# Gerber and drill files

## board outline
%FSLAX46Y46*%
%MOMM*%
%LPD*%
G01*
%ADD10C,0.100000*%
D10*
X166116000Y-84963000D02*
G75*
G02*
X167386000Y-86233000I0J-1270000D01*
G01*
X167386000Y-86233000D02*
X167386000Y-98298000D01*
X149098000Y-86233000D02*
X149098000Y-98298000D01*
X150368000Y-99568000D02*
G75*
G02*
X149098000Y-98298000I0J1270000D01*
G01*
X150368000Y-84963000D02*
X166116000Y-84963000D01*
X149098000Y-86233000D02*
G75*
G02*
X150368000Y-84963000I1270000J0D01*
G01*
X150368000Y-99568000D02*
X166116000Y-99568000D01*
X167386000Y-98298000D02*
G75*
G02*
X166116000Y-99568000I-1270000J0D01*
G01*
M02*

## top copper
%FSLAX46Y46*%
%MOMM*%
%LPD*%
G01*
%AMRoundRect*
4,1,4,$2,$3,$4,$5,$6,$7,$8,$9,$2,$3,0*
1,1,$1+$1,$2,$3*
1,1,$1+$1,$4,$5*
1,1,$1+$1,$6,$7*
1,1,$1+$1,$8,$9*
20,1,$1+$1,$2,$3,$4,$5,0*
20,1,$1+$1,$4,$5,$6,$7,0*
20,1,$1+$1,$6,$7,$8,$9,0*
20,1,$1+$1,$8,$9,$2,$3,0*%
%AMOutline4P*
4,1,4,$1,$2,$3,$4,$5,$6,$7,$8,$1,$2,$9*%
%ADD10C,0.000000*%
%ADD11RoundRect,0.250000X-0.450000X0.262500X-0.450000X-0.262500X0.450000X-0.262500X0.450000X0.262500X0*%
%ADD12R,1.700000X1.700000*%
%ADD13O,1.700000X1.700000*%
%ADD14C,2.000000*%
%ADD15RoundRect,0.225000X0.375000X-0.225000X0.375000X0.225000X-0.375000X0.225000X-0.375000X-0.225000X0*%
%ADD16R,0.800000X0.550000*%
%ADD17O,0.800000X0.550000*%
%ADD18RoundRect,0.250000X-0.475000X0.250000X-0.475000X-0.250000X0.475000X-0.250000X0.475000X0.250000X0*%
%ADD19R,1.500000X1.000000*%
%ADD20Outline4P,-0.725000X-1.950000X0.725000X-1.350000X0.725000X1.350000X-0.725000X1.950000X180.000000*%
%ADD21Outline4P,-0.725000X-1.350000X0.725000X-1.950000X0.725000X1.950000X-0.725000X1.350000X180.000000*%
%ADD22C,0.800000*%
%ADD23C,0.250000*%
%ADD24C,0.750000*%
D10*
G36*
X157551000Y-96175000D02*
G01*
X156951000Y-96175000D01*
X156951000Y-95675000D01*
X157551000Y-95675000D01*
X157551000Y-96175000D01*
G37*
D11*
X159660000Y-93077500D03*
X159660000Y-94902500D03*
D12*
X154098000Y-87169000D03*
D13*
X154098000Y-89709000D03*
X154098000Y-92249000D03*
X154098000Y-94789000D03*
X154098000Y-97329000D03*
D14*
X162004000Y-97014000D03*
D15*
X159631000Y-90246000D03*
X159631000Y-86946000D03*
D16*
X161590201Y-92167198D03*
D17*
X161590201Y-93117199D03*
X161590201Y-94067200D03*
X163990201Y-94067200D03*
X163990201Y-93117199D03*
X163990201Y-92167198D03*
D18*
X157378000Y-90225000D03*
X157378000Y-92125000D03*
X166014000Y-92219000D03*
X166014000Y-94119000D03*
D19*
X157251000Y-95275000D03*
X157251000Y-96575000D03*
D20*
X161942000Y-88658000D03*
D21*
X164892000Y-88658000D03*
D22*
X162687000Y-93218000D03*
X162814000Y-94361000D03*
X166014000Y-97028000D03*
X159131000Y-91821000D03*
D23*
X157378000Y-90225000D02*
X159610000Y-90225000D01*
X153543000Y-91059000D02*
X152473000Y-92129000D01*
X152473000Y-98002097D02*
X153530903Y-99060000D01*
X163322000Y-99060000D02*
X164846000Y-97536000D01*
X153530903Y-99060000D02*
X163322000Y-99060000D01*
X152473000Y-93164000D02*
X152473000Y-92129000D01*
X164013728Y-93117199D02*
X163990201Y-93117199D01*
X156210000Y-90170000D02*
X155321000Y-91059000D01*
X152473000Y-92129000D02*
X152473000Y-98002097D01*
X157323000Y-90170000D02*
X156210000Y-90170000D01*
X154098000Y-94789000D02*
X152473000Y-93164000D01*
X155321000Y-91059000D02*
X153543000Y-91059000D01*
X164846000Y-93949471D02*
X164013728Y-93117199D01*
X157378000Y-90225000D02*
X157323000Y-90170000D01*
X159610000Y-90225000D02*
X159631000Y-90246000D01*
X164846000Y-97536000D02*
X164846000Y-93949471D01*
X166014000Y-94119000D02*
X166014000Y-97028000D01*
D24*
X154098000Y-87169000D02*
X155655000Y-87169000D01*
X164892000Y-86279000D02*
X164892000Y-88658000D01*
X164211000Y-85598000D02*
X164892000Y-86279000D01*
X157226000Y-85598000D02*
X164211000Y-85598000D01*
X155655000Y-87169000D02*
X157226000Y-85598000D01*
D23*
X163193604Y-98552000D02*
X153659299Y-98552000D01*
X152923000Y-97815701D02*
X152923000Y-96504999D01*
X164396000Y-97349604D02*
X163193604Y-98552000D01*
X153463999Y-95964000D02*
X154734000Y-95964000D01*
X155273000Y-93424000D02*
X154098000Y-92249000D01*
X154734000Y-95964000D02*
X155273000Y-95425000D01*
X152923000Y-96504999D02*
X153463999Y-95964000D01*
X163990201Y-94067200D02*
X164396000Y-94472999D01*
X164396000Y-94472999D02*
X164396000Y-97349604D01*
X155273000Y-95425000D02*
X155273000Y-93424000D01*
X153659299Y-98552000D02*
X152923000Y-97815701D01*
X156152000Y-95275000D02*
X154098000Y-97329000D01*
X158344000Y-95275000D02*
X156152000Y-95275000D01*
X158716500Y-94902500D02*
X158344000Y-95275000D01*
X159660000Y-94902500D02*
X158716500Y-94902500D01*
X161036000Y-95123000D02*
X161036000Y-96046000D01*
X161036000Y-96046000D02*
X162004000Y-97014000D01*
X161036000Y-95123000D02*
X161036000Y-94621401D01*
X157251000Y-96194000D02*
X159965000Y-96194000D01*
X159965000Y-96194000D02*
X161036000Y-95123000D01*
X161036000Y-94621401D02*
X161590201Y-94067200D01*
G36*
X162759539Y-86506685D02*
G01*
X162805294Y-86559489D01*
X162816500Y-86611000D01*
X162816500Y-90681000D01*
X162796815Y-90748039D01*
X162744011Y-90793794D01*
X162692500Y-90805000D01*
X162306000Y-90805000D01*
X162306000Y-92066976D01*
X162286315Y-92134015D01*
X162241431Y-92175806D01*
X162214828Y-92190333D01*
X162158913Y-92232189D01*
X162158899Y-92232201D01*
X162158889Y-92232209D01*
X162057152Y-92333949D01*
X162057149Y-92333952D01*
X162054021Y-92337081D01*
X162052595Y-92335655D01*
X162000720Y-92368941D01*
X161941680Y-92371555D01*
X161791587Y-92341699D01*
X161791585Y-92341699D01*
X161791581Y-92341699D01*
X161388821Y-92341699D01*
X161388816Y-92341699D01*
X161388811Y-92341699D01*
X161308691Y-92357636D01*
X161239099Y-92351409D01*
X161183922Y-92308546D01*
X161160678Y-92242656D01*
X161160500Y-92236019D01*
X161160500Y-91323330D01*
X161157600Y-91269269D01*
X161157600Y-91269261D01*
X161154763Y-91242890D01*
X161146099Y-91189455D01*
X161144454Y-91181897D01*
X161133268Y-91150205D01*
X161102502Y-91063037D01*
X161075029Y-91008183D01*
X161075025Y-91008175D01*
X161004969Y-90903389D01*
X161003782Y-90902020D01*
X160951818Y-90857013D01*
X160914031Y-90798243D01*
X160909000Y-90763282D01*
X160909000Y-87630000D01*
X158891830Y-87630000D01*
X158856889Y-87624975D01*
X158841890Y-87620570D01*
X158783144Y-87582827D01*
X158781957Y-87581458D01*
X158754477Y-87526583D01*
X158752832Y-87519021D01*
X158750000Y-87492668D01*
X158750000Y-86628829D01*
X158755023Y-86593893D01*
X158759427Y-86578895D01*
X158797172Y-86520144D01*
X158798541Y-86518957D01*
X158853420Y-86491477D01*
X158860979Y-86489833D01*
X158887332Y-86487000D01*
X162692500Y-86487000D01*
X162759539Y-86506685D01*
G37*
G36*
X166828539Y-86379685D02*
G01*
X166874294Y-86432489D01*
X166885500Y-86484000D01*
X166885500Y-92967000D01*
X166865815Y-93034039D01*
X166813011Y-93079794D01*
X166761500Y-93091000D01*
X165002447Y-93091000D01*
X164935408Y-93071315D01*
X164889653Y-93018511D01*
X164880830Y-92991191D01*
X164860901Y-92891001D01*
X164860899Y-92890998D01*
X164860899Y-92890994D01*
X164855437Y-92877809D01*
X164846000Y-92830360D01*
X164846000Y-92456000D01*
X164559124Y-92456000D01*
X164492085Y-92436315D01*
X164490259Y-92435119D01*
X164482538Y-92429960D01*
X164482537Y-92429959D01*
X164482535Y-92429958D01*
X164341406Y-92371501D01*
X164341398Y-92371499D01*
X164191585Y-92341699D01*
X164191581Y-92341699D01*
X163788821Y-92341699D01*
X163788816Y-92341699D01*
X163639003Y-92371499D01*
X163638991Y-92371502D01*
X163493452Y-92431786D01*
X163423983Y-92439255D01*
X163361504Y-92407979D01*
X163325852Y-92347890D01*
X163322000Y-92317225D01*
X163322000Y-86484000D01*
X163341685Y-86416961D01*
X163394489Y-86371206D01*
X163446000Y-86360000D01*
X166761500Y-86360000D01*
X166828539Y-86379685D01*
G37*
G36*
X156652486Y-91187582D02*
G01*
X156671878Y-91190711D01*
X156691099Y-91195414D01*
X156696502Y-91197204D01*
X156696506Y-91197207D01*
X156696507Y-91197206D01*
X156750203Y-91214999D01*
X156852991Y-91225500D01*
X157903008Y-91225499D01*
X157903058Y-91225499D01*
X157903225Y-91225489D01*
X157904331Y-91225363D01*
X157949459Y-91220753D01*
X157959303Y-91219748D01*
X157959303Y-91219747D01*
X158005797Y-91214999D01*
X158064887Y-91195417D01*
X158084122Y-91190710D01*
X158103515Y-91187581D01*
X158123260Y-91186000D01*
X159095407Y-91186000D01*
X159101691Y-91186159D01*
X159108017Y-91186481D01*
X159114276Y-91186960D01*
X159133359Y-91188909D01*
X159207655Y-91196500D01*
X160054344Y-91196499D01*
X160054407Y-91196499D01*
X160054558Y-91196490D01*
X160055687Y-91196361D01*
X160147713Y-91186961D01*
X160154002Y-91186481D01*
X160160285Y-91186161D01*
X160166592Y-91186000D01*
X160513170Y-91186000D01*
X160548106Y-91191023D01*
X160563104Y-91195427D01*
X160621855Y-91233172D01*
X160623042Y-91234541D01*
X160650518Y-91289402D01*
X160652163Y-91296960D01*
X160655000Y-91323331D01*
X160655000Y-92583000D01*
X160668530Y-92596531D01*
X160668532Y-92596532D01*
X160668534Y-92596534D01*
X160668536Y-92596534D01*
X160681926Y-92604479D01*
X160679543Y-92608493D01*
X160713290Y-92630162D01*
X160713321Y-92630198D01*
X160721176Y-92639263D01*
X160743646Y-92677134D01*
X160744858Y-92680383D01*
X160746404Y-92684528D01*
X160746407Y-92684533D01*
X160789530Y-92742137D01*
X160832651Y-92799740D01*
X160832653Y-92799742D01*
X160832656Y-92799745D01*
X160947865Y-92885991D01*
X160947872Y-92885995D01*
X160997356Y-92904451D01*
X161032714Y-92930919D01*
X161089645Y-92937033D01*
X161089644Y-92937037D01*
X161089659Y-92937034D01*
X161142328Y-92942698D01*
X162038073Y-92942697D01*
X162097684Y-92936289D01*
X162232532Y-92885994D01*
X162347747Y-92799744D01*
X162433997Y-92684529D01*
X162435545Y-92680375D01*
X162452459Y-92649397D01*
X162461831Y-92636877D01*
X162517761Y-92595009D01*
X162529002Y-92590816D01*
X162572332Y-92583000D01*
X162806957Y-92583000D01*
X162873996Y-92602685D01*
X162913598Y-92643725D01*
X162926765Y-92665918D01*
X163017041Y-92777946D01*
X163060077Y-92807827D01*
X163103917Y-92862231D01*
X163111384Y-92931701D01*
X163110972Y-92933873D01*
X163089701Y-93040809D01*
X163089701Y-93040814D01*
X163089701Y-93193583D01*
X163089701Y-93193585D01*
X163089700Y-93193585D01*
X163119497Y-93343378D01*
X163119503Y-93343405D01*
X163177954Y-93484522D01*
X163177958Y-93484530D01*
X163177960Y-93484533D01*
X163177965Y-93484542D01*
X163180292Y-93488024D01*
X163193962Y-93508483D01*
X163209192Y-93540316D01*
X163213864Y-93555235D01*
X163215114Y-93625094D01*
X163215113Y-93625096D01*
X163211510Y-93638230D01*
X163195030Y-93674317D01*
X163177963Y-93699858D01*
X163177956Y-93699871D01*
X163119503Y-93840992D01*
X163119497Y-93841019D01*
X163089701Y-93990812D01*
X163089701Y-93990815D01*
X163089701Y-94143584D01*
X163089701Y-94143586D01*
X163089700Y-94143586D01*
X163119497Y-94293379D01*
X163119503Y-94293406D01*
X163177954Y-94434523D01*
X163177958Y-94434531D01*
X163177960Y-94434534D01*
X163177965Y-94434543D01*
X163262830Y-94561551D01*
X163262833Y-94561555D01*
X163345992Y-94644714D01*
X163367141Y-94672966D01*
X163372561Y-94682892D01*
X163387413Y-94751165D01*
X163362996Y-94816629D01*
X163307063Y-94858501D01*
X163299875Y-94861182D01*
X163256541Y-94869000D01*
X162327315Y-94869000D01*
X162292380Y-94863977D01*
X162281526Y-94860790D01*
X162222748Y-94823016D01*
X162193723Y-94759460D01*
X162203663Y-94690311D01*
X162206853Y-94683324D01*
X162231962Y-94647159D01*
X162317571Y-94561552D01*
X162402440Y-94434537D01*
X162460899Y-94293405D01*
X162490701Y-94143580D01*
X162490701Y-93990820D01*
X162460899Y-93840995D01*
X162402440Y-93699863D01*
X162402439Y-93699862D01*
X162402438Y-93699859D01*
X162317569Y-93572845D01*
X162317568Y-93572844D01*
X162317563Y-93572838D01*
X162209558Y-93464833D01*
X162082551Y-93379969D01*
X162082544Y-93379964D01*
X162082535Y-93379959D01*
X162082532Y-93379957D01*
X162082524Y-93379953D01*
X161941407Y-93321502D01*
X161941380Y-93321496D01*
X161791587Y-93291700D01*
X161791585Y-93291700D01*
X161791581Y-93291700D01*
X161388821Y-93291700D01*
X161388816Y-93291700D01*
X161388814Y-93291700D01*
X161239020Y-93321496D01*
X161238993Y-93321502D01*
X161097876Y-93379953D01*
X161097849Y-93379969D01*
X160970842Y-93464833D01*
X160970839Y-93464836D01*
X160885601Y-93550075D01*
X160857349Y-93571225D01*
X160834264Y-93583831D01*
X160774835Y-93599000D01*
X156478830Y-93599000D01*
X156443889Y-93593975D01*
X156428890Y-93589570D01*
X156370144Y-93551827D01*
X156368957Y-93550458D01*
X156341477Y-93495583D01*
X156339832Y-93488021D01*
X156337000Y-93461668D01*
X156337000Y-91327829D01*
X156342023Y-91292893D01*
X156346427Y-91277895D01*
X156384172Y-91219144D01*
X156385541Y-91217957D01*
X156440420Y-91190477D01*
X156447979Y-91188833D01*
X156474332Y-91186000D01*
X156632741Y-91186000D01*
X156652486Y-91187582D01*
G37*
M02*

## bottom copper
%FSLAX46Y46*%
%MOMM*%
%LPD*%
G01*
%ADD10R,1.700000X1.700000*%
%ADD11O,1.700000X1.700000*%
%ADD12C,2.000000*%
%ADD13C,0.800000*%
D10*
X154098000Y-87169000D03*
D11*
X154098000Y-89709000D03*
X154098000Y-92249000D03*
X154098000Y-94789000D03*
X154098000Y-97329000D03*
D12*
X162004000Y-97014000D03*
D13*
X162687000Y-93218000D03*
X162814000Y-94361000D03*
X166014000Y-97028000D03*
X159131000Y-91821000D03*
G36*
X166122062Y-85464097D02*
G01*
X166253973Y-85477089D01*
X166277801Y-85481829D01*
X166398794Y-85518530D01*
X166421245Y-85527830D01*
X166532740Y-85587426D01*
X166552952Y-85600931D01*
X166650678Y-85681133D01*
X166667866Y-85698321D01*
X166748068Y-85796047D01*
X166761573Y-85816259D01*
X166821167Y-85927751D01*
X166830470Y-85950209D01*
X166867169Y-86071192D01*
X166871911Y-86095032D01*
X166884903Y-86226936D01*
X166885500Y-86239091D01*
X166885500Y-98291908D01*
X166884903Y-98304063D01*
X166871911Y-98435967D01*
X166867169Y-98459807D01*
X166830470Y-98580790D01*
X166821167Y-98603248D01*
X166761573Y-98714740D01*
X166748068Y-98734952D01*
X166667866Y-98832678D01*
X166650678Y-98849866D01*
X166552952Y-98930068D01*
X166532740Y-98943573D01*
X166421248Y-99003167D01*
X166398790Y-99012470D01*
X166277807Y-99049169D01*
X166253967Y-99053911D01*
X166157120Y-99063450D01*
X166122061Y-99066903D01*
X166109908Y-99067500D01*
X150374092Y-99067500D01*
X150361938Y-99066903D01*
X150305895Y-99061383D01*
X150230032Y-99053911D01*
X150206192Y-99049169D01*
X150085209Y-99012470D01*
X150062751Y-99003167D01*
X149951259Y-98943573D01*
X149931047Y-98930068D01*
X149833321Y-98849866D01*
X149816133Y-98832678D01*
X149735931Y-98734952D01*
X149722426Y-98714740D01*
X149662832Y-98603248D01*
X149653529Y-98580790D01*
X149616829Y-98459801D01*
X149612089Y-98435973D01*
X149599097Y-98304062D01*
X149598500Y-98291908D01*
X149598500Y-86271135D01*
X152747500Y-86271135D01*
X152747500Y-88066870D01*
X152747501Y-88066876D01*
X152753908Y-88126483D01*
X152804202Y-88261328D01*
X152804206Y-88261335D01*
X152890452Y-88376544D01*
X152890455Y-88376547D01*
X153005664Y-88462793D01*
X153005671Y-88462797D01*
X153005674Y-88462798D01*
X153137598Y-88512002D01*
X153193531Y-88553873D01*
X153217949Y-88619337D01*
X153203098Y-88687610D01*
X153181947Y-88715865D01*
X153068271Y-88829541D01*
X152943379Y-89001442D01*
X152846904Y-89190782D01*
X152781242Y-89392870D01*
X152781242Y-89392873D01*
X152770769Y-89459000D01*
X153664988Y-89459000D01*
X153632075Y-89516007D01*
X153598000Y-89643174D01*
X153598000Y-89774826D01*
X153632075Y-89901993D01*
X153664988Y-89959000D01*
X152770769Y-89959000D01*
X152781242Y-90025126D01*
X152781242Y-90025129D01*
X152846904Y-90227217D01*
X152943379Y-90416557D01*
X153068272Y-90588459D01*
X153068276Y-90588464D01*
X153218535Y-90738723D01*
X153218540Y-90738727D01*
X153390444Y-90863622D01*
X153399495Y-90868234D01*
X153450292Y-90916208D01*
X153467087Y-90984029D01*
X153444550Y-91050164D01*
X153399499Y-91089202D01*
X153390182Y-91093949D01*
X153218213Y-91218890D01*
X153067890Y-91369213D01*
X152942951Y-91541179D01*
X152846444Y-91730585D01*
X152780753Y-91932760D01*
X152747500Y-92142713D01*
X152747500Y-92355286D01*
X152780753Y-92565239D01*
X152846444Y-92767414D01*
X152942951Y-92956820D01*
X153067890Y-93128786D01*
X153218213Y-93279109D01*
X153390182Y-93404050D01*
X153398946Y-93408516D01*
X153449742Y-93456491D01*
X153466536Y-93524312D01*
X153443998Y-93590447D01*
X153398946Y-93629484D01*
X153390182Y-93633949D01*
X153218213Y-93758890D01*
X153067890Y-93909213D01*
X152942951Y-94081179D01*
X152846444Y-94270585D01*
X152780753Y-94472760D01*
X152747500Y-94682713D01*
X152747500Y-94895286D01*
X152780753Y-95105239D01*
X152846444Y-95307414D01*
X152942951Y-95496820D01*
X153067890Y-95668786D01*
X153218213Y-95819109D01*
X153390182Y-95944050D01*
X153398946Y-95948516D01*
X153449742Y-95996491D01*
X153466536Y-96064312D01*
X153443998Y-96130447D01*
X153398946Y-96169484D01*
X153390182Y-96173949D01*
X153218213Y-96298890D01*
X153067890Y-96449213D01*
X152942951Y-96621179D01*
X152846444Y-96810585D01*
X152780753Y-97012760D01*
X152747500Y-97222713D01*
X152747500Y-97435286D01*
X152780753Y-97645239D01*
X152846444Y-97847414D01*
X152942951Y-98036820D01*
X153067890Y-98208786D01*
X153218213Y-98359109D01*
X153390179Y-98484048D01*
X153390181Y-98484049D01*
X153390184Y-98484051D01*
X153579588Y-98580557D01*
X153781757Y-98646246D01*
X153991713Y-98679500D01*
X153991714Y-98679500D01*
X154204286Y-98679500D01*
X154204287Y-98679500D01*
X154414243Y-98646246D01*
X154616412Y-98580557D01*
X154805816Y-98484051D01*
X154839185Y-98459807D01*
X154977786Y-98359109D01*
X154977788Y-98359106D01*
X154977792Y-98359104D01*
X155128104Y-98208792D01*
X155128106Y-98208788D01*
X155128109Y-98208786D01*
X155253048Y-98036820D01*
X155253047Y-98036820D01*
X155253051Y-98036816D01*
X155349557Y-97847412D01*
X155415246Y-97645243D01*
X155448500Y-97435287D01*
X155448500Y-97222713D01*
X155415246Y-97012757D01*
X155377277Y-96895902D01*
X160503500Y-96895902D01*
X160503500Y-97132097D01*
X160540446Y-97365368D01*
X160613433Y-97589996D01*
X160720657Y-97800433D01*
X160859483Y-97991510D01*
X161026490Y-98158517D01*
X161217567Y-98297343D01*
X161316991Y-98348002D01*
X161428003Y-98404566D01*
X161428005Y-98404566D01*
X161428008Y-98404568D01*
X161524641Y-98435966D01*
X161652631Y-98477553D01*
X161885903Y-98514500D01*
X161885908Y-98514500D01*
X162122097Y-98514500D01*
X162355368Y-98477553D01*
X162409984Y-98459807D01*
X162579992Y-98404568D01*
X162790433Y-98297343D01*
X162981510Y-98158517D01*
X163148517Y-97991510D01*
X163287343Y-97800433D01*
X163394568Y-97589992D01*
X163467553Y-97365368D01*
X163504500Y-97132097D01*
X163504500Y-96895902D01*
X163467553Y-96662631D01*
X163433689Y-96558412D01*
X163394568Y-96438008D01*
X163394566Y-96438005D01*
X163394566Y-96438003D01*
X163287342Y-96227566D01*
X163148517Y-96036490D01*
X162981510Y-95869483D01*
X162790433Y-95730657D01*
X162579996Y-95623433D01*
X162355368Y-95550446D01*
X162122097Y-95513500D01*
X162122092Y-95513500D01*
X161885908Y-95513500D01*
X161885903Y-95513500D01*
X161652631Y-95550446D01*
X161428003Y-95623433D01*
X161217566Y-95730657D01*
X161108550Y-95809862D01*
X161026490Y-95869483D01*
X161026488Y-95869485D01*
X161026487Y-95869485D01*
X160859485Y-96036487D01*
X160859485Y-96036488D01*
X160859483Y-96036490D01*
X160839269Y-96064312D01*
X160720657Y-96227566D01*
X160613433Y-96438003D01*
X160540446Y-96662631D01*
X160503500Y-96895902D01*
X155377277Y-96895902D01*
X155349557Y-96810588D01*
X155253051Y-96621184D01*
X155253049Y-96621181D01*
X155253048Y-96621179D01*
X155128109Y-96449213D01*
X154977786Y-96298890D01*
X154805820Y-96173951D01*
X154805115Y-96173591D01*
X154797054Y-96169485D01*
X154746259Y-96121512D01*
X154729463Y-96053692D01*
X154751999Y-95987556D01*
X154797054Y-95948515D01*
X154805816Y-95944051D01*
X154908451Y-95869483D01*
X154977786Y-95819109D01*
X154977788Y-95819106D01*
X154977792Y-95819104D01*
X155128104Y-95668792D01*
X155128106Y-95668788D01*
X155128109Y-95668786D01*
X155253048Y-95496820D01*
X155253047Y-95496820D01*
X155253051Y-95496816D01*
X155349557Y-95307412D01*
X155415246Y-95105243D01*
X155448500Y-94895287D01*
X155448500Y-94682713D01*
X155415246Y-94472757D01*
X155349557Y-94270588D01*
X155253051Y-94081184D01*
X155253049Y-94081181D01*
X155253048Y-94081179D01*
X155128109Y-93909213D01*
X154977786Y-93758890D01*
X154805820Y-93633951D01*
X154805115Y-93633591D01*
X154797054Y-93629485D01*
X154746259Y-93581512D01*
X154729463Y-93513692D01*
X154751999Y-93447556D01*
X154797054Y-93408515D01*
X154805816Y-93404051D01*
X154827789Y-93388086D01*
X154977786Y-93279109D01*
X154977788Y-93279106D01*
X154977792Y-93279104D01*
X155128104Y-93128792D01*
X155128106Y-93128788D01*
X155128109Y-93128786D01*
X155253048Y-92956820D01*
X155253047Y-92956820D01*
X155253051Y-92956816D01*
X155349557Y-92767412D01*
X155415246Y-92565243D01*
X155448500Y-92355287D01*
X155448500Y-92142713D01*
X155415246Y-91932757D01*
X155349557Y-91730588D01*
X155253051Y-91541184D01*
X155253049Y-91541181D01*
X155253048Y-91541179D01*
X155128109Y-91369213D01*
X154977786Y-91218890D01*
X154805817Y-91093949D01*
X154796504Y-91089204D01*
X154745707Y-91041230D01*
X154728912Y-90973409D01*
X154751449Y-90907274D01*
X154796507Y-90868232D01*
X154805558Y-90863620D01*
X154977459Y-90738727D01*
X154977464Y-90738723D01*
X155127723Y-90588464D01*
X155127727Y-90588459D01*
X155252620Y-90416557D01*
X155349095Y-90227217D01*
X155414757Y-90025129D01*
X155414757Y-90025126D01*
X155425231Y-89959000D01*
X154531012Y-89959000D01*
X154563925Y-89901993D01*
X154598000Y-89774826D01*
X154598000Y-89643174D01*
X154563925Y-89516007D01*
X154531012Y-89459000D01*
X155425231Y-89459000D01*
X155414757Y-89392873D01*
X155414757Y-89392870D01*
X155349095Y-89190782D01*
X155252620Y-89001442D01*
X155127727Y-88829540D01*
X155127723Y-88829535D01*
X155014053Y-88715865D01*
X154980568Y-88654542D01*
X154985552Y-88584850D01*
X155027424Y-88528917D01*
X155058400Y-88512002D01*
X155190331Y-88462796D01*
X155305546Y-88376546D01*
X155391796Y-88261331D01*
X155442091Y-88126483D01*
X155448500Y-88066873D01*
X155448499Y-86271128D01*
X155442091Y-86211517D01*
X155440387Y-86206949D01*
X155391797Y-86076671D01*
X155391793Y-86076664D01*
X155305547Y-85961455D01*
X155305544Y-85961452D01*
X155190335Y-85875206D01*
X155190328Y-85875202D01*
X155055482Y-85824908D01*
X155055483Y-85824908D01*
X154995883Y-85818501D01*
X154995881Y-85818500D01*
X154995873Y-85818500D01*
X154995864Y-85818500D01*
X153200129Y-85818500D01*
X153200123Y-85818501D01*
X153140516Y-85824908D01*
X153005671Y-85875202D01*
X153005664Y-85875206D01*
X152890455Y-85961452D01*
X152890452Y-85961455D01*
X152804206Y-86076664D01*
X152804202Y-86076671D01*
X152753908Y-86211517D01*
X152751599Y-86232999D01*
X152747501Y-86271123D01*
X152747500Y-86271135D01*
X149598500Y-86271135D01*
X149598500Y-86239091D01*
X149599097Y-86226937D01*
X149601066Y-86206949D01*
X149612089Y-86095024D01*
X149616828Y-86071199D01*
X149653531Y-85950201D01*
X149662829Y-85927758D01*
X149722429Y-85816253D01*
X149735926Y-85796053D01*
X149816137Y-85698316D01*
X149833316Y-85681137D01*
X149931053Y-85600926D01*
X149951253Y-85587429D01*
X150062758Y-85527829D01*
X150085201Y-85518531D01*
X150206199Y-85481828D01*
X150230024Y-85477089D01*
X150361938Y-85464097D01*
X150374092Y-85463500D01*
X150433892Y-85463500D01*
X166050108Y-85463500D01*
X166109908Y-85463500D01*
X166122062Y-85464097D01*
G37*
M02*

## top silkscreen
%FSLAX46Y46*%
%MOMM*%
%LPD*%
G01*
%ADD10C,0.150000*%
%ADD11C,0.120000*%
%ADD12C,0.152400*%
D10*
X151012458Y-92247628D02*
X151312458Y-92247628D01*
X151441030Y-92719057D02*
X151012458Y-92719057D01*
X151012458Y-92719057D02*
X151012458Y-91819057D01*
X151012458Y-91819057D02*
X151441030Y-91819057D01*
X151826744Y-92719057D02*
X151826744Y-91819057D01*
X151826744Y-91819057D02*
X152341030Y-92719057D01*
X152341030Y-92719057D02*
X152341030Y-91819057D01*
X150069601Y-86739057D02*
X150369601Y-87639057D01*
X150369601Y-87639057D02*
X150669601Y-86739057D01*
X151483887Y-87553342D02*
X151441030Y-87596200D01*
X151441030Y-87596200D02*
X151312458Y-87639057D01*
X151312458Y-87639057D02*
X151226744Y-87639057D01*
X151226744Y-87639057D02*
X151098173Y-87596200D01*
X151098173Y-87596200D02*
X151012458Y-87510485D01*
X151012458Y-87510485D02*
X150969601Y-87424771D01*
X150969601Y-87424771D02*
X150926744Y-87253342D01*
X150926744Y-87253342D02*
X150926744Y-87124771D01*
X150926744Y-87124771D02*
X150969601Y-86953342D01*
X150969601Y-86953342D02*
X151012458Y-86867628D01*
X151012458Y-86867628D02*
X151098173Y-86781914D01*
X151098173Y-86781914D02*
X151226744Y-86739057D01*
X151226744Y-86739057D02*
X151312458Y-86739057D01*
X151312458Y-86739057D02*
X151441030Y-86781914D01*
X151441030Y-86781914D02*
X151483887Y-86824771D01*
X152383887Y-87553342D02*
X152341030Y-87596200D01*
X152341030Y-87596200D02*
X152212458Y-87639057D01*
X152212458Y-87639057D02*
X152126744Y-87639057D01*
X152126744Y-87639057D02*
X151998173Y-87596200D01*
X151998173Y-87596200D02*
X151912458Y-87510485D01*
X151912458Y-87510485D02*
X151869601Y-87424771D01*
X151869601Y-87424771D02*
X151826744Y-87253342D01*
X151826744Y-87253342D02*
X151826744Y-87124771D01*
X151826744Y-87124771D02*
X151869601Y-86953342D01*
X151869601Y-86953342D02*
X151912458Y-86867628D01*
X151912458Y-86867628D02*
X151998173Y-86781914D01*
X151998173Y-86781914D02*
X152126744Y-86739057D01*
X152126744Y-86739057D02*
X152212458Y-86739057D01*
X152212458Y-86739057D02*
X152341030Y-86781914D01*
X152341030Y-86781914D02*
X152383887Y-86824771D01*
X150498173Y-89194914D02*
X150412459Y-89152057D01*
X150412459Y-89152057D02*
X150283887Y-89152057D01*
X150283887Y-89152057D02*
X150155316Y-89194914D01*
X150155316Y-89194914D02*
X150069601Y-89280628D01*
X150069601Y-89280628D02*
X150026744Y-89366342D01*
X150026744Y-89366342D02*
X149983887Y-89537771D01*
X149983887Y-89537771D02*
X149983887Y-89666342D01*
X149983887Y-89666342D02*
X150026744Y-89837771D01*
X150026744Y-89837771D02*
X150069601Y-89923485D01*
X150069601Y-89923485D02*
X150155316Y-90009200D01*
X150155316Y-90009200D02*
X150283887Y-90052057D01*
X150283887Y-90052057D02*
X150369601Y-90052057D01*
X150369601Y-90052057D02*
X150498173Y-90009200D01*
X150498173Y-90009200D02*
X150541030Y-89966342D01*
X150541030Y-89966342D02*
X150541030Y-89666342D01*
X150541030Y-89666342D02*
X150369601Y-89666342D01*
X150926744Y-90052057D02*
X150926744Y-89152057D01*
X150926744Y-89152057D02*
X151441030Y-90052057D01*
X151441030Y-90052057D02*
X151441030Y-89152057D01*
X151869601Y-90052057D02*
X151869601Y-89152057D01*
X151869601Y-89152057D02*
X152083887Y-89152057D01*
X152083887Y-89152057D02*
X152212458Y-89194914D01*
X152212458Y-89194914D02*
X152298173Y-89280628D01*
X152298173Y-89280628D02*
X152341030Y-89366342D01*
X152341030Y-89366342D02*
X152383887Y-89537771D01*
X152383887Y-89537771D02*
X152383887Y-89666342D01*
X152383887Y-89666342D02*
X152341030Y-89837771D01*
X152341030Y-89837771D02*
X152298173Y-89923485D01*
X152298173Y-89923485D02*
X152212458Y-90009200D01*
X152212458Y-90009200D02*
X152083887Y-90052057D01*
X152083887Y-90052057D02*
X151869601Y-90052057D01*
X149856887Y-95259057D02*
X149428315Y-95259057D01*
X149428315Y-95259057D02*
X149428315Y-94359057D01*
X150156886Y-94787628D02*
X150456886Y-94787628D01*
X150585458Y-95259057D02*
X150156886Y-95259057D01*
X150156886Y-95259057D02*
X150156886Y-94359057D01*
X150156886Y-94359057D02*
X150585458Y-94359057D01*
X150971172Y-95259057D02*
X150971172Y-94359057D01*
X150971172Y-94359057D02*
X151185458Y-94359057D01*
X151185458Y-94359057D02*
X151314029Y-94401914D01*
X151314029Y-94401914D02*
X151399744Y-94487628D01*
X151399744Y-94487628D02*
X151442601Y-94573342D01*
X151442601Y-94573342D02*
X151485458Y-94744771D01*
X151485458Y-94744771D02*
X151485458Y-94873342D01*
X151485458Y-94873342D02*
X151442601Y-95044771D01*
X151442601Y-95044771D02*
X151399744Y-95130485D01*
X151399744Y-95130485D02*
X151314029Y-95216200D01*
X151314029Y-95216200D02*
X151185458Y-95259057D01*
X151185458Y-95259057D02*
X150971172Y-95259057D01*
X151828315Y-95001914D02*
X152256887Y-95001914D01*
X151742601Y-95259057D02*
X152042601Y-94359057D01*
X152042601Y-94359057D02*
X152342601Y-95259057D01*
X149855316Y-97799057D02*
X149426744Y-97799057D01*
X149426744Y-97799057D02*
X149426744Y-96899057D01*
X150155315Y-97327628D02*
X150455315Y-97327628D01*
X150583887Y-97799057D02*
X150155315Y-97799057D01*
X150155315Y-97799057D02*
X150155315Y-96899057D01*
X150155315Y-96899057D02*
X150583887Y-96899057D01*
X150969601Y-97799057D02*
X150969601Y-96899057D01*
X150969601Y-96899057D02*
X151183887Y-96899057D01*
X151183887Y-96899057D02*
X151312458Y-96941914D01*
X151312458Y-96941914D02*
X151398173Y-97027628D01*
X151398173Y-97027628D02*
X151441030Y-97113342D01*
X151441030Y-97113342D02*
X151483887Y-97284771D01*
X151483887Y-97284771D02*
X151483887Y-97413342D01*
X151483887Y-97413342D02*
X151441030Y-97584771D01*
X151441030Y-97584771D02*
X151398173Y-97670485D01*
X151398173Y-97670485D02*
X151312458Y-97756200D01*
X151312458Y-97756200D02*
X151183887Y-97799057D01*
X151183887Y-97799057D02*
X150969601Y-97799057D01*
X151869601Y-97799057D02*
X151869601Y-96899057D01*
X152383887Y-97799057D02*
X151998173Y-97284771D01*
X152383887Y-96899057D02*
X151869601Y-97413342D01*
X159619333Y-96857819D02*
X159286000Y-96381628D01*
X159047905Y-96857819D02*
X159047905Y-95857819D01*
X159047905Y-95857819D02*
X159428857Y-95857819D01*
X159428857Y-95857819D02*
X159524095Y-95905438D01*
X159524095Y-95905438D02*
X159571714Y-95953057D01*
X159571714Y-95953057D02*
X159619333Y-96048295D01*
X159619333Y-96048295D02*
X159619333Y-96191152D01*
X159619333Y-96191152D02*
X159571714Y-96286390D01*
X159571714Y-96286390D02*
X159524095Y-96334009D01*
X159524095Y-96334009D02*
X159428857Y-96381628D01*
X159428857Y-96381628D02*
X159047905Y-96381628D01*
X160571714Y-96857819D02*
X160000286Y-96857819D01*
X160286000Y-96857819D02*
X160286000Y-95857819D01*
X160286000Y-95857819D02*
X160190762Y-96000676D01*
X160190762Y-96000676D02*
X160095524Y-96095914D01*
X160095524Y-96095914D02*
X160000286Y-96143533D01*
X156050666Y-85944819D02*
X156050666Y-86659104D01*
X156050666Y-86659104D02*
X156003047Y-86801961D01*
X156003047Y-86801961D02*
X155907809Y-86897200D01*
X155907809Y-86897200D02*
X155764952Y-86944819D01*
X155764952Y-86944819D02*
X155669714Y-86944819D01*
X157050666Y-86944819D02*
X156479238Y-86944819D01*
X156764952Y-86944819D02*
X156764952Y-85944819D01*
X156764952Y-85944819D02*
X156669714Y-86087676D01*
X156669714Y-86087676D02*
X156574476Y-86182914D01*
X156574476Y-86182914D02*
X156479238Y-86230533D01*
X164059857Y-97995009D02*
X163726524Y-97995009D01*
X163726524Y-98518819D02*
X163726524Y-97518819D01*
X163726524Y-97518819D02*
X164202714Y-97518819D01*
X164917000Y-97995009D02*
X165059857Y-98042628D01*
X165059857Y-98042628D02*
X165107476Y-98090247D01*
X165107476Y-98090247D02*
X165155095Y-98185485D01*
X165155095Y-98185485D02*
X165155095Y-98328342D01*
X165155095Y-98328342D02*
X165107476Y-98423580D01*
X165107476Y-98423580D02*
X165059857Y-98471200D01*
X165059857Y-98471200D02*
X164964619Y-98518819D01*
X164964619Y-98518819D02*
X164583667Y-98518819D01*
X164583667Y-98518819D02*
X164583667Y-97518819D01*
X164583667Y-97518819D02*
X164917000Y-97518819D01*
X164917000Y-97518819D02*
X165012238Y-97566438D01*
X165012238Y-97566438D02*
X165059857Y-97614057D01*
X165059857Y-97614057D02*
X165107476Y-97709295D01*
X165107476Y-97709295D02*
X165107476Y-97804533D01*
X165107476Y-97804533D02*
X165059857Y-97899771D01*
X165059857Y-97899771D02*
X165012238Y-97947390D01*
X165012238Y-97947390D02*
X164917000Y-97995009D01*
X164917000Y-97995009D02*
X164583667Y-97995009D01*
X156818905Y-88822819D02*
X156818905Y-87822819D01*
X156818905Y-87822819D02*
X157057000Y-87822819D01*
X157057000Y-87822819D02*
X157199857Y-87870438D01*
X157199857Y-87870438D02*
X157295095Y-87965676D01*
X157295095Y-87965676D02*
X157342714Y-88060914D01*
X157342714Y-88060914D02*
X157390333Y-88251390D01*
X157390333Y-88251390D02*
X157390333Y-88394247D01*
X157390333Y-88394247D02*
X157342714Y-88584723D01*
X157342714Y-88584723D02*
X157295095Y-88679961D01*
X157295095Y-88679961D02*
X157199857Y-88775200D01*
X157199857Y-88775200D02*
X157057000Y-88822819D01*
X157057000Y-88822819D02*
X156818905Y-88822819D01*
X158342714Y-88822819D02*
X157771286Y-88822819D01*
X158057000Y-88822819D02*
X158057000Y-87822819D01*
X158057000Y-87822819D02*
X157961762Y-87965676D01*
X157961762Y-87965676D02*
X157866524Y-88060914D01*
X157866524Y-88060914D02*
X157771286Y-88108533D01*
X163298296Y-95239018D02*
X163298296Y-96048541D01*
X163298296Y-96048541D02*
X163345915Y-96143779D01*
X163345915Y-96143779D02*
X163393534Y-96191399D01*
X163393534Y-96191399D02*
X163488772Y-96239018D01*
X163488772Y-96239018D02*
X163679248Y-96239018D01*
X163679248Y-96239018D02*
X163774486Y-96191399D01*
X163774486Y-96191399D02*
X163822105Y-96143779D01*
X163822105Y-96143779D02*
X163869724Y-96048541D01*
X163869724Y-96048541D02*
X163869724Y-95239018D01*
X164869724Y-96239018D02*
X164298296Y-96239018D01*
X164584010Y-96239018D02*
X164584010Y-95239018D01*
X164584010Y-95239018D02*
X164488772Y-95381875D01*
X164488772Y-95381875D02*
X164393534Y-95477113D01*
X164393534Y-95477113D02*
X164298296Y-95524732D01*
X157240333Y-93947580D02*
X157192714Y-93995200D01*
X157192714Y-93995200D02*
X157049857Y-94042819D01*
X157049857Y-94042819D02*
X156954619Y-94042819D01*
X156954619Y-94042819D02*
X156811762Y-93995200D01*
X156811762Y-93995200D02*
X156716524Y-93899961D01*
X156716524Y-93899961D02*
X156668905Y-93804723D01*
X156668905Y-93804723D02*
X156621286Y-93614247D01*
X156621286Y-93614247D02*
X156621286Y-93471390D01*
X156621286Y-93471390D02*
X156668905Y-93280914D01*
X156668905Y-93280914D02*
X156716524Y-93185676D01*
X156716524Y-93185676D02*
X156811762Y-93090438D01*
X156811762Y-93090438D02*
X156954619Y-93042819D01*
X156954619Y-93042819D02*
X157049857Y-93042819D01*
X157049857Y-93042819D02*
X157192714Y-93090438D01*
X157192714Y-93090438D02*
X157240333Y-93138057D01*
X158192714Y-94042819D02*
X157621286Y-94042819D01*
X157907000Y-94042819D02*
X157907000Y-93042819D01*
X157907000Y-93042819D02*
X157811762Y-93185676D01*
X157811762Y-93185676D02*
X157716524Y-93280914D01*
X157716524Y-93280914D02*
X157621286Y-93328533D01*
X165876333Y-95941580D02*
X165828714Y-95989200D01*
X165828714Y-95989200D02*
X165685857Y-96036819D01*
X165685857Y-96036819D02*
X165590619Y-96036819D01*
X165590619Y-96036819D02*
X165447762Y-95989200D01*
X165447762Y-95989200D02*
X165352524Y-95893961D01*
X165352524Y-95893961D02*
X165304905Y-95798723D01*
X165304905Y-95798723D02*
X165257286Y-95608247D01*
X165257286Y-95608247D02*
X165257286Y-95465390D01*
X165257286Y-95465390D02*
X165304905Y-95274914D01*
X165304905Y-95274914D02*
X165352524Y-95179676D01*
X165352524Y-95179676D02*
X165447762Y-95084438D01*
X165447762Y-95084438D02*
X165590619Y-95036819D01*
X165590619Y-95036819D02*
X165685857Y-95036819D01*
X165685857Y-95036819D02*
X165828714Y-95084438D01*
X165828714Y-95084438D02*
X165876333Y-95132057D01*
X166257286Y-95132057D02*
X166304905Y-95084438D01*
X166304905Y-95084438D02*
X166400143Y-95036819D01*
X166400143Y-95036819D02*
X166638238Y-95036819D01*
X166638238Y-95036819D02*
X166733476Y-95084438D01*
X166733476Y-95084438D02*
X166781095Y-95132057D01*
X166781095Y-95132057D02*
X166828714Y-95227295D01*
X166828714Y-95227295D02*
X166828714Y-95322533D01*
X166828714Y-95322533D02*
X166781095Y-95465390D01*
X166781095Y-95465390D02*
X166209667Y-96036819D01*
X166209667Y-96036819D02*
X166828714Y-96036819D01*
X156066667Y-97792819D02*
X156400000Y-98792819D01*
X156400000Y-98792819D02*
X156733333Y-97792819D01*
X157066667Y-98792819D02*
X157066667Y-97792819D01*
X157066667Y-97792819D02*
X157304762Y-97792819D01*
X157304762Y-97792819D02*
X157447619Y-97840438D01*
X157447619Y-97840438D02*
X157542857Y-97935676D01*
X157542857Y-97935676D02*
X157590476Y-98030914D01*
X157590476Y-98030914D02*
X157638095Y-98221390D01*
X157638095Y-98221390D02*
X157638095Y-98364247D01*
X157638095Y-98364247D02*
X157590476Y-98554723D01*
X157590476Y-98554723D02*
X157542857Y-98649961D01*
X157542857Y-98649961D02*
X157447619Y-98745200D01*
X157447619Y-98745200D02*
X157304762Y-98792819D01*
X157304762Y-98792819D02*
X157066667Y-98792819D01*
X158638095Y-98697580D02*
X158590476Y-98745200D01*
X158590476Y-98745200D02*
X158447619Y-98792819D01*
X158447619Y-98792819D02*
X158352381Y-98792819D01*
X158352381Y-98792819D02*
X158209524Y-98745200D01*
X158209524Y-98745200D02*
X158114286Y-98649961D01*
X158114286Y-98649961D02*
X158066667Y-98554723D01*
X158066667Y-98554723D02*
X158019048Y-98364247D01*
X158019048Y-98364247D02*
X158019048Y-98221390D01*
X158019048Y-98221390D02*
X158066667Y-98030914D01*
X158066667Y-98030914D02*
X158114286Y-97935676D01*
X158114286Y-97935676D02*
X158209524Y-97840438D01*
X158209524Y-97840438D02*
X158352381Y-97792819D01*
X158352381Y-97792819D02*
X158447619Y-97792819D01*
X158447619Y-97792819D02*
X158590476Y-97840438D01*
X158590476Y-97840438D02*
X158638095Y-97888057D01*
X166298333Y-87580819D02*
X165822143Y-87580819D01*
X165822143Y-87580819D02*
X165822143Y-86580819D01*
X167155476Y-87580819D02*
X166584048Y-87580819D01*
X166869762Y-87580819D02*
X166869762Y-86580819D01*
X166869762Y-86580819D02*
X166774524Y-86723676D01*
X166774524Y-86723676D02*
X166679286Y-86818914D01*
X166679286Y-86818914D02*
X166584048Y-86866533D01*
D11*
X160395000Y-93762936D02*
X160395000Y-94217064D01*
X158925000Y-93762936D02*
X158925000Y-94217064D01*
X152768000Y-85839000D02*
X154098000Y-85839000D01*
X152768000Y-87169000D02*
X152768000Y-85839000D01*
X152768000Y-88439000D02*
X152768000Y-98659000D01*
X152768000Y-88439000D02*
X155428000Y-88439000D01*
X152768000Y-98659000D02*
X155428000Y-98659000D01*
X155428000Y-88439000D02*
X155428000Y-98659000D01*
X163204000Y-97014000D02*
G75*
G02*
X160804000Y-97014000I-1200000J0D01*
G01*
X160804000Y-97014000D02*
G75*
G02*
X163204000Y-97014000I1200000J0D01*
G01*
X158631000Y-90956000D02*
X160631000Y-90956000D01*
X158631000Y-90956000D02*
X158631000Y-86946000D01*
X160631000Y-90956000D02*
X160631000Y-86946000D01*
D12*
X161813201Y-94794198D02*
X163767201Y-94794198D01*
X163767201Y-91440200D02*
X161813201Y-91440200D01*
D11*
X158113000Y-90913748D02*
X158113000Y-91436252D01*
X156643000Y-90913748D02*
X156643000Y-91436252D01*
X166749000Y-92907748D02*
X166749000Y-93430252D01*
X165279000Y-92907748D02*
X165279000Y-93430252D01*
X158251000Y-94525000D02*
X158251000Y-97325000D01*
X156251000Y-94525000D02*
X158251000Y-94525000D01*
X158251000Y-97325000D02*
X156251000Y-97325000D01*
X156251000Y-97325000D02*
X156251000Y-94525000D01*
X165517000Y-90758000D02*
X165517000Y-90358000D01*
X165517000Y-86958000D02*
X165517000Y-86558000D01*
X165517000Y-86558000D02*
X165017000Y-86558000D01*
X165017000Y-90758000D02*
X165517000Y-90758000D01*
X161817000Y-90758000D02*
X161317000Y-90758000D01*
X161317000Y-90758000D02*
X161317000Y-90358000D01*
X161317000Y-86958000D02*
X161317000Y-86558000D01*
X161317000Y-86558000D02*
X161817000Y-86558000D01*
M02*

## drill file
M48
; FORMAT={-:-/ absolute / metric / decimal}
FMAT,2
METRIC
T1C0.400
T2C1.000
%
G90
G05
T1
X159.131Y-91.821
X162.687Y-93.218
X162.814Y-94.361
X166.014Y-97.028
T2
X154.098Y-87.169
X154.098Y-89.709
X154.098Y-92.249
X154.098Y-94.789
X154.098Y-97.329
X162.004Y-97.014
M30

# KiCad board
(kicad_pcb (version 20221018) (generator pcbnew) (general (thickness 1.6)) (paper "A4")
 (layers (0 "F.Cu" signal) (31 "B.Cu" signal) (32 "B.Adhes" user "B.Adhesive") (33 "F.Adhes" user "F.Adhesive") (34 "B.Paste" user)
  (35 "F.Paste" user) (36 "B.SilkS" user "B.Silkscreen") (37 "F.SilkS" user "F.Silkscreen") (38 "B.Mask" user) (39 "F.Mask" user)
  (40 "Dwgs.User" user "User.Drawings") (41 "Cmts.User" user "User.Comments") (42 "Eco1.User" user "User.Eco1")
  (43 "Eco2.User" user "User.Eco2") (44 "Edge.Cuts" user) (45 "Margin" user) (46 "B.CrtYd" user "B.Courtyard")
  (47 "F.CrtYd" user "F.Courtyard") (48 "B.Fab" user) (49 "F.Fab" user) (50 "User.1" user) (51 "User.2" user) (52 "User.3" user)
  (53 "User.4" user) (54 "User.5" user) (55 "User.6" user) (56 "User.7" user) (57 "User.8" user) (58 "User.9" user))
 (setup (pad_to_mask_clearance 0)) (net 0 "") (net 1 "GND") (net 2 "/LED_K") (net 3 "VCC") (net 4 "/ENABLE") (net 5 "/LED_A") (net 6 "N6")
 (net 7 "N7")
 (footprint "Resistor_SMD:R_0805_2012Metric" (layer "F.Cu") (at 159.66 93.99 -90)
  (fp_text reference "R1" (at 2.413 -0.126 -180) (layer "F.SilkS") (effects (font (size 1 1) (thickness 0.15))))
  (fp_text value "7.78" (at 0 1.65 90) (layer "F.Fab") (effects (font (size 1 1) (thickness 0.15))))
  (fp_line (start -0.227064 -0.735) (end 0.227064 -0.735) (stroke (width 0.12) (type solid)) (layer "F.SilkS"))
  (fp_line (start -0.227064 0.735) (end 0.227064 0.735) (stroke (width 0.12) (type solid)) (layer "F.SilkS"))
  (pad "1" smd roundrect (at -0.9125 0 270) (size 1.025 1.4) (layers "F.Cu" "F.Paste" "F.Mask") (roundrect_rratio 0.243902439) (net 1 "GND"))
  (pad "2" smd roundrect (at 0.9125 0 270) (size 1.025 1.4) (layers "F.Cu" "F.Paste" "F.Mask") (roundrect_rratio 0.243902439)
   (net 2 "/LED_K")))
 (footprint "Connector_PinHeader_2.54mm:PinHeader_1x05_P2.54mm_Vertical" (layer "F.Cu") (at 154.098 87.169)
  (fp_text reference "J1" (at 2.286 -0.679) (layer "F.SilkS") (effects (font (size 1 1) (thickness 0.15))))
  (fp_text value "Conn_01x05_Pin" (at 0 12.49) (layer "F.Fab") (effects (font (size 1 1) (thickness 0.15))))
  (fp_line (start -1.33 -1.33) (end 0 -1.33) (stroke (width 0.12) (type solid)) (layer "F.SilkS"))
  (fp_line (start -1.33 0) (end -1.33 -1.33) (stroke (width 0.12) (type solid)) (layer "F.SilkS"))
  (fp_line (start -1.33 1.27) (end -1.33 11.49) (stroke (width 0.12) (type solid)) (layer "F.SilkS"))
  (fp_line (start -1.33 1.27) (end 1.33 1.27) (stroke (width 0.12) (type solid)) (layer "F.SilkS"))
  (fp_line (start -1.33 11.49) (end 1.33 11.49) (stroke (width 0.12) (type solid)) (layer "F.SilkS"))
  (fp_line (start 1.33 1.27) (end 1.33 11.49) (stroke (width 0.12) (type solid)) (layer "F.SilkS"))
  (pad "1" thru_hole rect (at 0 0) (size 1.7 1.7) (drill 1) (layers "*.Cu" "*.Mask") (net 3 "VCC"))
  (pad "2" thru_hole oval (at 0 2.54) (size 1.7 1.7) (drill 1) (layers "*.Cu" "*.Mask") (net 1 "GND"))
  (pad "3" thru_hole oval (at 0 5.08) (size 1.7 1.7) (drill 1) (layers "*.Cu" "*.Mask") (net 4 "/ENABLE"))
  (pad "4" thru_hole oval (at 0 7.62) (size 1.7 1.7) (drill 1) (layers "*.Cu" "*.Mask") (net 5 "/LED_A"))
  (pad "5" thru_hole oval (at 0 10.16) (size 1.7 1.7) (drill 1) (layers "*.Cu" "*.Mask") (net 2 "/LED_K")))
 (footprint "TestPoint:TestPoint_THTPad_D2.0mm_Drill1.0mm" (layer "F.Cu") (at 162.004 97.014)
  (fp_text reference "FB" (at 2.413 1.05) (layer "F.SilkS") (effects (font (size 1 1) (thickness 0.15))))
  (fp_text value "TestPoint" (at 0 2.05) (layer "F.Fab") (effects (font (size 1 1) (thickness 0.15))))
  (fp_circle (center 0 0) (end 0 1.2) (stroke (width 0.12) (type solid)) (fill none) (layer "F.SilkS"))
  (pad "1" thru_hole circle (at 0 0) (size 2 2) (drill 1) (layers "*.Cu" "*.Mask") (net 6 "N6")))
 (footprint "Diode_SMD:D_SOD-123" (layer "F.Cu") (at 159.631 88.596 90)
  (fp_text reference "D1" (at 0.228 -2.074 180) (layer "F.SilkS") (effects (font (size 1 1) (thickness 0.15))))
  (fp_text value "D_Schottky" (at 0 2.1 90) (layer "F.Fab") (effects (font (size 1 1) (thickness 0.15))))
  (fp_line (start -2.36 -1) (end -2.36 1) (stroke (width 0.12) (type solid)) (layer "F.SilkS"))
  (fp_line (start -2.36 -1) (end 1.65 -1) (stroke (width 0.12) (type solid)) (layer "F.SilkS"))
  (fp_line (start -2.36 1) (end 1.65 1) (stroke (width 0.12) (type solid)) (layer "F.SilkS"))
  (pad "1" smd roundrect (at -1.65 0 90) (size 0.9 1.2) (layers "F.Cu" "F.Paste" "F.Mask") (roundrect_rratio 0.25) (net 5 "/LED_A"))
  (pad "2" smd roundrect (at 1.65 0 90) (size 0.9 1.2) (layers "F.Cu" "F.Paste" "F.Mask") (roundrect_rratio 0.25) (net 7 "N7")))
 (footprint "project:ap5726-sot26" (layer "F.Cu") (at 162.790201 93.117199)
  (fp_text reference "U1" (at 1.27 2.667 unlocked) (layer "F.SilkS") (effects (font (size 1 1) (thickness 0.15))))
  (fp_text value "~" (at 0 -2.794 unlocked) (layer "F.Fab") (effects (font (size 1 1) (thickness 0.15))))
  (fp_line (start -0.977 1.676999) (end 0.977 1.676999) (stroke (width 0.1524) (type solid)) (layer "F.SilkS"))
  (fp_line (start 0.977 -1.676999) (end -0.977 -1.676999) (stroke (width 0.1524) (type solid)) (layer "F.SilkS"))
  (pad "1" smd rect (at -1.2 -0.950001) (size 0.8 0.55) (layers "F.Cu" "F.Paste" "F.Mask") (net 7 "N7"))
  (pad "2" smd oval (at -1.2 0) (size 0.8 0.55) (layers "F.Cu" "F.Paste" "F.Mask") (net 1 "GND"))
  (pad "3" smd oval (at -1.2 0.950001) (size 0.8 0.55) (layers "F.Cu" "F.Paste" "F.Mask") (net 6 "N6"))
  (pad "4" smd oval (at 1.2 0.950001) (size 0.8 0.55) (layers "F.Cu" "F.Paste" "F.Mask") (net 4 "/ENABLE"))
  (pad "5" smd oval (at 1.2 0) (size 0.8 0.55) (layers "F.Cu" "F.Paste" "F.Mask") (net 5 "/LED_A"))
  (pad "6" smd oval (at 1.2 -0.950001) (size 0.8 0.55) (layers "F.Cu" "F.Paste" "F.Mask") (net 3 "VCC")))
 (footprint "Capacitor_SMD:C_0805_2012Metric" (layer "F.Cu") (at 157.378 91.175 -90)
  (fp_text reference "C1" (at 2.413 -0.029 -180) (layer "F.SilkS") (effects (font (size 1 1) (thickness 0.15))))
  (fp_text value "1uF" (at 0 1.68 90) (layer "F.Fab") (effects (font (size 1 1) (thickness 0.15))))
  (fp_line (start -0.261252 -0.735) (end 0.261252 -0.735) (stroke (width 0.12) (type solid)) (layer "F.SilkS"))
  (fp_line (start -0.261252 0.735) (end 0.261252 0.735) (stroke (width 0.12) (type solid)) (layer "F.SilkS"))
  (pad "1" smd roundrect (at -0.95 0 270) (size 1 1.45) (layers "F.Cu" "F.Paste" "F.Mask") (roundrect_rratio 0.25) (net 5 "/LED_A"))
  (pad "2" smd roundrect (at 0.95 0 270) (size 1 1.45) (layers "F.Cu" "F.Paste" "F.Mask") (roundrect_rratio 0.25) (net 1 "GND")))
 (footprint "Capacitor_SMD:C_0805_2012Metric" (layer "F.Cu") (at 166.014 93.169 -90)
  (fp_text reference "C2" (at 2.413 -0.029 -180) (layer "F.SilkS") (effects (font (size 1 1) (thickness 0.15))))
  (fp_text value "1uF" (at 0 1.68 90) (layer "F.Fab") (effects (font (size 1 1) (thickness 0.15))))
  (fp_line (start -0.261252 -0.735) (end 0.261252 -0.735) (stroke (width 0.12) (type solid)) (layer "F.SilkS"))
  (fp_line (start -0.261252 0.735) (end 0.261252 0.735) (stroke (width 0.12) (type solid)) (layer "F.SilkS"))
  (pad "1" smd roundrect (at -0.95 0 270) (size 1 1.45) (layers "F.Cu" "F.Paste" "F.Mask") (roundrect_rratio 0.25) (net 3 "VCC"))
  (pad "2" smd roundrect (at 0.95 0 270) (size 1 1.45) (layers "F.Cu" "F.Paste" "F.Mask") (roundrect_rratio 0.25) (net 1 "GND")))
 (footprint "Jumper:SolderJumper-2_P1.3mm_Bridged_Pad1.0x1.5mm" (layer "F.Cu") (at 157.251 95.925 -90) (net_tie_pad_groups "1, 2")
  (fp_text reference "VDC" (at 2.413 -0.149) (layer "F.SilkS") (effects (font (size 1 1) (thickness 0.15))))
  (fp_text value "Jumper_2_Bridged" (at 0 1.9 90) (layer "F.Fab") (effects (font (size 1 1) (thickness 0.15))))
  (fp_poly (pts (xy -0.25 -0.3) (xy 0.25 -0.3) (xy 0.25 0.3) (xy -0.25 0.3)) (stroke (width 0) (type solid)) (fill solid) (layer "F.Cu"))
  (fp_line (start -1.4 -1) (end 1.4 -1) (stroke (width 0.12) (type solid)) (layer "F.SilkS"))
  (fp_line (start -1.4 1) (end -1.4 -1) (stroke (width 0.12) (type solid)) (layer "F.SilkS"))
  (fp_line (start 1.4 -1) (end 1.4 1) (stroke (width 0.12) (type solid)) (layer "F.SilkS"))
  (fp_line (start 1.4 1) (end -1.4 1) (stroke (width 0.12) (type solid)) (layer "F.SilkS"))
  (pad "1" smd rect (at -0.65 0 270) (size 1 1.5) (layers "F.Cu" "F.Mask") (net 2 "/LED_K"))
  (pad "2" smd rect (at 0.65 0 270) (size 1 1.5) (layers "F.Cu" "F.Mask") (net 6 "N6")))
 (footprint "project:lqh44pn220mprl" (layer "F.Cu") (at 163.417 88.658 180)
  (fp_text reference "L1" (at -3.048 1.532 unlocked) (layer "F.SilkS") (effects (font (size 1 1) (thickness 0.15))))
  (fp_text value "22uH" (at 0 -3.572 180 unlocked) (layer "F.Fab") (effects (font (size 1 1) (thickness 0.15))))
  (fp_line (start -2.1 -2.1) (end -2.1 -1.7) (stroke (width 0.12) (type default)) (layer "F.SilkS"))
  (fp_line (start -2.1 1.7) (end -2.1 2.1) (stroke (width 0.12) (type default)) (layer "F.SilkS"))
  (fp_line (start -2.1 2.1) (end -1.6 2.1) (stroke (width 0.12) (type default)) (layer "F.SilkS"))
  (fp_line (start -1.6 -2.1) (end -2.1 -2.1) (stroke (width 0.12) (type default)) (layer "F.SilkS"))
  (fp_line (start 1.6 -2.1) (end 2.1 -2.1) (stroke (width 0.12) (type default)) (layer "F.SilkS"))
  (fp_line (start 2.1 -2.1) (end 2.1 -1.7) (stroke (width 0.12) (type default)) (layer "F.SilkS"))
  (fp_line (start 2.1 1.7) (end 2.1 2.1) (stroke (width 0.12) (type default)) (layer "F.SilkS"))
  (fp_line (start 2.1 2.1) (end 1.6 2.1) (stroke (width 0.12) (type default)) (layer "F.SilkS"))
  (pad "1" smd trapezoid (at 1.475 0 180) (size 1.45 3.3) (rect_delta 0.6 0) (layers "F.Cu" "F.Paste" "F.Mask") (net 7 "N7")
   (thermal_bridge_angle 45))
  (pad "2" smd trapezoid (at -1.475 0 180) (size 1.45 3.3) (rect_delta -0.6 0) (layers "F.Cu" "F.Paste" "F.Mask") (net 3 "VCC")
   (thermal_bridge_angle 45)))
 (gr_arc (start 166.116 84.963) (mid 167.014026 85.334974) (end 167.386 86.233) (stroke (width 0.1) (type default)) (layer "Edge.Cuts"))
 (gr_line (start 167.386 86.233) (end 167.386 98.298) (stroke (width 0.1) (type default)) (layer "Edge.Cuts"))
 (gr_line (start 149.098 86.233) (end 149.098 98.298) (stroke (width 0.1) (type default)) (layer "Edge.Cuts"))
 (gr_arc (start 150.368 99.568) (mid 149.469974 99.196026) (end 149.098 98.298) (stroke (width 0.1) (type default)) (layer "Edge.Cuts"))
 (gr_line (start 150.368 84.963) (end 166.116 84.963) (stroke (width 0.1) (type default)) (layer "Edge.Cuts"))
 (gr_arc (start 149.098 86.233) (mid 149.469974 85.334974) (end 150.368 84.963) (stroke (width 0.1) (type default)) (layer "Edge.Cuts"))
 (gr_line (start 150.368 99.568) (end 166.116 99.568) (stroke (width 0.1) (type default)) (layer "Edge.Cuts"))
 (gr_arc (start 167.386 98.298) (mid 167.014026 99.196026) (end 166.116 99.568) (stroke (width 0.1) (type default)) (layer "Edge.Cuts"))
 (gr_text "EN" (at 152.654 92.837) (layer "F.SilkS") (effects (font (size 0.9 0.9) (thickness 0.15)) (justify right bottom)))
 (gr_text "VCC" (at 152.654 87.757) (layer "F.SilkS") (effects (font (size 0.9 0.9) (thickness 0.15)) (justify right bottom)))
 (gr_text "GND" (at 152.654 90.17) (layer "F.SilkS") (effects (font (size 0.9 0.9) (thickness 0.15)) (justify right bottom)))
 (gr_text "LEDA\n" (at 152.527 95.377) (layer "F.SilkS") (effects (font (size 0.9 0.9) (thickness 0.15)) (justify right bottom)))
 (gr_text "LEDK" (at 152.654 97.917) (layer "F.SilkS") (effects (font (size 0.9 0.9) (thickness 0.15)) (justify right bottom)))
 (segment (start 157.378 90.225) (end 159.61 90.225) (width 0.25) (layer "F.Cu") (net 5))
 (segment (start 153.543 91.059) (end 152.473 92.129) (width 0.25) (layer "F.Cu") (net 5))
 (segment (start 152.473 98.002097) (end 153.530903 99.06) (width 0.25) (layer "F.Cu") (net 5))
 (segment (start 163.322 99.06) (end 164.846 97.536) (width 0.25) (layer "F.Cu") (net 5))
 (segment (start 153.530903 99.06) (end 163.322 99.06) (width 0.25) (layer "F.Cu") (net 5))
 (segment (start 152.473 93.164) (end 152.473 92.129) (width 0.25) (layer "F.Cu") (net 5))
 (segment (start 164.013728 93.117199) (end 163.990201 93.117199) (width 0.25) (layer "F.Cu") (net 5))
 (segment (start 156.21 90.17) (end 155.321 91.059) (width 0.25) (layer "F.Cu") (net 5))
 (segment (start 152.473 92.129) (end 152.473 98.002097) (width 0.25) (layer "F.Cu") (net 5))
 (segment (start 157.323 90.17) (end 156.21 90.17) (width 0.25) (layer "F.Cu") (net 5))
 (segment (start 154.098 94.789) (end 152.473 93.164) (width 0.25) (layer "F.Cu") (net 5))
 (segment (start 155.321 91.059) (end 153.543 91.059) (width 0.25) (layer "F.Cu") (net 5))
 (segment (start 164.846 93.949471) (end 164.013728 93.117199) (width 0.25) (layer "F.Cu") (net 5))
 (segment (start 157.378 90.225) (end 157.323 90.17) (width 0.25) (layer "F.Cu") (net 5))
 (segment (start 159.61 90.225) (end 159.631 90.246) (width 0.25) (layer "F.Cu") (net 5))
 (segment (start 164.846 97.536) (end 164.846 93.949471) (width 0.25) (layer "F.Cu") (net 5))
 (segment (start 166.014 94.119) (end 166.014 97.028) (width 0.25) (layer "F.Cu") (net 1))
 (via (at 162.687 93.218) (size 0.8) (drill 0.4) (layers "F.Cu" "B.Cu") (free) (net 1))
 (via (at 162.814 94.361) (size 0.8) (drill 0.4) (layers "F.Cu" "B.Cu") (free) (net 1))
 (via (at 166.014 97.028) (size 0.8) (drill 0.4) (layers "F.Cu" "B.Cu") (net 1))
 (via (at 159.131 91.821) (size 0.8) (drill 0.4) (layers "F.Cu" "B.Cu") (free) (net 1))
 (segment (start 154.098 87.169) (end 155.655 87.169) (width 0.75) (layer "F.Cu") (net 3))
 (segment (start 164.892 86.279) (end 164.892 88.658) (width 0.75) (layer "F.Cu") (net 3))
 (segment (start 164.211 85.598) (end 164.892 86.279) (width 0.75) (layer "F.Cu") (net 3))
 (segment (start 157.226 85.598) (end 164.211 85.598) (width 0.75) (layer "F.Cu") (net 3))
 (segment (start 155.655 87.169) (end 157.226 85.598) (width 0.75) (layer "F.Cu") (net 3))
 (segment (start 163.193604 98.552) (end 153.659299 98.552) (width 0.25) (layer "F.Cu") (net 4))
 (segment (start 152.923 97.815701) (end 152.923 96.504999) (width 0.25) (layer "F.Cu") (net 4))
 (segment (start 164.396 97.349604) (end 163.193604 98.552) (width 0.25) (layer "F.Cu") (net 4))
 (segment (start 153.463999 95.964) (end 154.734 95.964) (width 0.25) (layer "F.Cu") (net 4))
 (segment (start 155.273 93.424) (end 154.098 92.249) (width 0.25) (layer "F.Cu") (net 4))
 (segment (start 154.734 95.964) (end 155.273 95.425) (width 0.25) (layer "F.Cu") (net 4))
 (segment (start 152.923 96.504999) (end 153.463999 95.964) (width 0.25) (layer "F.Cu") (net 4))
 (segment (start 163.990201 94.0672) (end 164.396 94.472999) (width 0.25) (layer "F.Cu") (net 4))
 (segment (start 164.396 94.472999) (end 164.396 97.349604) (width 0.25) (layer "F.Cu") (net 4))
 (segment (start 155.273 95.425) (end 155.273 93.424) (width 0.25) (layer "F.Cu") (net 4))
 (segment (start 153.659299 98.552) (end 152.923 97.815701) (width 0.25) (layer "F.Cu") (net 4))
 (segment (start 156.152 95.275) (end 154.098 97.329) (width 0.25) (layer "F.Cu") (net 2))
 (segment (start 158.344 95.275) (end 156.152 95.275) (width 0.25) (layer "F.Cu") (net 2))
 (segment (start 158.7165 94.9025) (end 158.344 95.275) (width 0.25) (layer "F.Cu") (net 2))
 (segment (start 159.66 94.9025) (end 158.7165 94.9025) (width 0.25) (layer "F.Cu") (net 2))
 (segment (start 161.036 95.123) (end 161.036 96.046) (width 0.25) (layer "F.Cu") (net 6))
 (segment (start 161.036 96.046) (end 162.004 97.014) (width 0.25) (layer "F.Cu") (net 6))
 (segment (start 161.036 95.123) (end 161.036 94.621401) (width 0.25) (layer "F.Cu") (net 6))
 (segment (start 157.251 96.194) (end 159.965 96.194) (width 0.25) (layer "F.Cu") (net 6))
 (segment (start 159.965 96.194) (end 161.036 95.123) (width 0.25) (layer "F.Cu") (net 6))
 (segment (start 161.036 94.621401) (end 161.590201 94.0672) (width 0.25) (layer "F.Cu") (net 6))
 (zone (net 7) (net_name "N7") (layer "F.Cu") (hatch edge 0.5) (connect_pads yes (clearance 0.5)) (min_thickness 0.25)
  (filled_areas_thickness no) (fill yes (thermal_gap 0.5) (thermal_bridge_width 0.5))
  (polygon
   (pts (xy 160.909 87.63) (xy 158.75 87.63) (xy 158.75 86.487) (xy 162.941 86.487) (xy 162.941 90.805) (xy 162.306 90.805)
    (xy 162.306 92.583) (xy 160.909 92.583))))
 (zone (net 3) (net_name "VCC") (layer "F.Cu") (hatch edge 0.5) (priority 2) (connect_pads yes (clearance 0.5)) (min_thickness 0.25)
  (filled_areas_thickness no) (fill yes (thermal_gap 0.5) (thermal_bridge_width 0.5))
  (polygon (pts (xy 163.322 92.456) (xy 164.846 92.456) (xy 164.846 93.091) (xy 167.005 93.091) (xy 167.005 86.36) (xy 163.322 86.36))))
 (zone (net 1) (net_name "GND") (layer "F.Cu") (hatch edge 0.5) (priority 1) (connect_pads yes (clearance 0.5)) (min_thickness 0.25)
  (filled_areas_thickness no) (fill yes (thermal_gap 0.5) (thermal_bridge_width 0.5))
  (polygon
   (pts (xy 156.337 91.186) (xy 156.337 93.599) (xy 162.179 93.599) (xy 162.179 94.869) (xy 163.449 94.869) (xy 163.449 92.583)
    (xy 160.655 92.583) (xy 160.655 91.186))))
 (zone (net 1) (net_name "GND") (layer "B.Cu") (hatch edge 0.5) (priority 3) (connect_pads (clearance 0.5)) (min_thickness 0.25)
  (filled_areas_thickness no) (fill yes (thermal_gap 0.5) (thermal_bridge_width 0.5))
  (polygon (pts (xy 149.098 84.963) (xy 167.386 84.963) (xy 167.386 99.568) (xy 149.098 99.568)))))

